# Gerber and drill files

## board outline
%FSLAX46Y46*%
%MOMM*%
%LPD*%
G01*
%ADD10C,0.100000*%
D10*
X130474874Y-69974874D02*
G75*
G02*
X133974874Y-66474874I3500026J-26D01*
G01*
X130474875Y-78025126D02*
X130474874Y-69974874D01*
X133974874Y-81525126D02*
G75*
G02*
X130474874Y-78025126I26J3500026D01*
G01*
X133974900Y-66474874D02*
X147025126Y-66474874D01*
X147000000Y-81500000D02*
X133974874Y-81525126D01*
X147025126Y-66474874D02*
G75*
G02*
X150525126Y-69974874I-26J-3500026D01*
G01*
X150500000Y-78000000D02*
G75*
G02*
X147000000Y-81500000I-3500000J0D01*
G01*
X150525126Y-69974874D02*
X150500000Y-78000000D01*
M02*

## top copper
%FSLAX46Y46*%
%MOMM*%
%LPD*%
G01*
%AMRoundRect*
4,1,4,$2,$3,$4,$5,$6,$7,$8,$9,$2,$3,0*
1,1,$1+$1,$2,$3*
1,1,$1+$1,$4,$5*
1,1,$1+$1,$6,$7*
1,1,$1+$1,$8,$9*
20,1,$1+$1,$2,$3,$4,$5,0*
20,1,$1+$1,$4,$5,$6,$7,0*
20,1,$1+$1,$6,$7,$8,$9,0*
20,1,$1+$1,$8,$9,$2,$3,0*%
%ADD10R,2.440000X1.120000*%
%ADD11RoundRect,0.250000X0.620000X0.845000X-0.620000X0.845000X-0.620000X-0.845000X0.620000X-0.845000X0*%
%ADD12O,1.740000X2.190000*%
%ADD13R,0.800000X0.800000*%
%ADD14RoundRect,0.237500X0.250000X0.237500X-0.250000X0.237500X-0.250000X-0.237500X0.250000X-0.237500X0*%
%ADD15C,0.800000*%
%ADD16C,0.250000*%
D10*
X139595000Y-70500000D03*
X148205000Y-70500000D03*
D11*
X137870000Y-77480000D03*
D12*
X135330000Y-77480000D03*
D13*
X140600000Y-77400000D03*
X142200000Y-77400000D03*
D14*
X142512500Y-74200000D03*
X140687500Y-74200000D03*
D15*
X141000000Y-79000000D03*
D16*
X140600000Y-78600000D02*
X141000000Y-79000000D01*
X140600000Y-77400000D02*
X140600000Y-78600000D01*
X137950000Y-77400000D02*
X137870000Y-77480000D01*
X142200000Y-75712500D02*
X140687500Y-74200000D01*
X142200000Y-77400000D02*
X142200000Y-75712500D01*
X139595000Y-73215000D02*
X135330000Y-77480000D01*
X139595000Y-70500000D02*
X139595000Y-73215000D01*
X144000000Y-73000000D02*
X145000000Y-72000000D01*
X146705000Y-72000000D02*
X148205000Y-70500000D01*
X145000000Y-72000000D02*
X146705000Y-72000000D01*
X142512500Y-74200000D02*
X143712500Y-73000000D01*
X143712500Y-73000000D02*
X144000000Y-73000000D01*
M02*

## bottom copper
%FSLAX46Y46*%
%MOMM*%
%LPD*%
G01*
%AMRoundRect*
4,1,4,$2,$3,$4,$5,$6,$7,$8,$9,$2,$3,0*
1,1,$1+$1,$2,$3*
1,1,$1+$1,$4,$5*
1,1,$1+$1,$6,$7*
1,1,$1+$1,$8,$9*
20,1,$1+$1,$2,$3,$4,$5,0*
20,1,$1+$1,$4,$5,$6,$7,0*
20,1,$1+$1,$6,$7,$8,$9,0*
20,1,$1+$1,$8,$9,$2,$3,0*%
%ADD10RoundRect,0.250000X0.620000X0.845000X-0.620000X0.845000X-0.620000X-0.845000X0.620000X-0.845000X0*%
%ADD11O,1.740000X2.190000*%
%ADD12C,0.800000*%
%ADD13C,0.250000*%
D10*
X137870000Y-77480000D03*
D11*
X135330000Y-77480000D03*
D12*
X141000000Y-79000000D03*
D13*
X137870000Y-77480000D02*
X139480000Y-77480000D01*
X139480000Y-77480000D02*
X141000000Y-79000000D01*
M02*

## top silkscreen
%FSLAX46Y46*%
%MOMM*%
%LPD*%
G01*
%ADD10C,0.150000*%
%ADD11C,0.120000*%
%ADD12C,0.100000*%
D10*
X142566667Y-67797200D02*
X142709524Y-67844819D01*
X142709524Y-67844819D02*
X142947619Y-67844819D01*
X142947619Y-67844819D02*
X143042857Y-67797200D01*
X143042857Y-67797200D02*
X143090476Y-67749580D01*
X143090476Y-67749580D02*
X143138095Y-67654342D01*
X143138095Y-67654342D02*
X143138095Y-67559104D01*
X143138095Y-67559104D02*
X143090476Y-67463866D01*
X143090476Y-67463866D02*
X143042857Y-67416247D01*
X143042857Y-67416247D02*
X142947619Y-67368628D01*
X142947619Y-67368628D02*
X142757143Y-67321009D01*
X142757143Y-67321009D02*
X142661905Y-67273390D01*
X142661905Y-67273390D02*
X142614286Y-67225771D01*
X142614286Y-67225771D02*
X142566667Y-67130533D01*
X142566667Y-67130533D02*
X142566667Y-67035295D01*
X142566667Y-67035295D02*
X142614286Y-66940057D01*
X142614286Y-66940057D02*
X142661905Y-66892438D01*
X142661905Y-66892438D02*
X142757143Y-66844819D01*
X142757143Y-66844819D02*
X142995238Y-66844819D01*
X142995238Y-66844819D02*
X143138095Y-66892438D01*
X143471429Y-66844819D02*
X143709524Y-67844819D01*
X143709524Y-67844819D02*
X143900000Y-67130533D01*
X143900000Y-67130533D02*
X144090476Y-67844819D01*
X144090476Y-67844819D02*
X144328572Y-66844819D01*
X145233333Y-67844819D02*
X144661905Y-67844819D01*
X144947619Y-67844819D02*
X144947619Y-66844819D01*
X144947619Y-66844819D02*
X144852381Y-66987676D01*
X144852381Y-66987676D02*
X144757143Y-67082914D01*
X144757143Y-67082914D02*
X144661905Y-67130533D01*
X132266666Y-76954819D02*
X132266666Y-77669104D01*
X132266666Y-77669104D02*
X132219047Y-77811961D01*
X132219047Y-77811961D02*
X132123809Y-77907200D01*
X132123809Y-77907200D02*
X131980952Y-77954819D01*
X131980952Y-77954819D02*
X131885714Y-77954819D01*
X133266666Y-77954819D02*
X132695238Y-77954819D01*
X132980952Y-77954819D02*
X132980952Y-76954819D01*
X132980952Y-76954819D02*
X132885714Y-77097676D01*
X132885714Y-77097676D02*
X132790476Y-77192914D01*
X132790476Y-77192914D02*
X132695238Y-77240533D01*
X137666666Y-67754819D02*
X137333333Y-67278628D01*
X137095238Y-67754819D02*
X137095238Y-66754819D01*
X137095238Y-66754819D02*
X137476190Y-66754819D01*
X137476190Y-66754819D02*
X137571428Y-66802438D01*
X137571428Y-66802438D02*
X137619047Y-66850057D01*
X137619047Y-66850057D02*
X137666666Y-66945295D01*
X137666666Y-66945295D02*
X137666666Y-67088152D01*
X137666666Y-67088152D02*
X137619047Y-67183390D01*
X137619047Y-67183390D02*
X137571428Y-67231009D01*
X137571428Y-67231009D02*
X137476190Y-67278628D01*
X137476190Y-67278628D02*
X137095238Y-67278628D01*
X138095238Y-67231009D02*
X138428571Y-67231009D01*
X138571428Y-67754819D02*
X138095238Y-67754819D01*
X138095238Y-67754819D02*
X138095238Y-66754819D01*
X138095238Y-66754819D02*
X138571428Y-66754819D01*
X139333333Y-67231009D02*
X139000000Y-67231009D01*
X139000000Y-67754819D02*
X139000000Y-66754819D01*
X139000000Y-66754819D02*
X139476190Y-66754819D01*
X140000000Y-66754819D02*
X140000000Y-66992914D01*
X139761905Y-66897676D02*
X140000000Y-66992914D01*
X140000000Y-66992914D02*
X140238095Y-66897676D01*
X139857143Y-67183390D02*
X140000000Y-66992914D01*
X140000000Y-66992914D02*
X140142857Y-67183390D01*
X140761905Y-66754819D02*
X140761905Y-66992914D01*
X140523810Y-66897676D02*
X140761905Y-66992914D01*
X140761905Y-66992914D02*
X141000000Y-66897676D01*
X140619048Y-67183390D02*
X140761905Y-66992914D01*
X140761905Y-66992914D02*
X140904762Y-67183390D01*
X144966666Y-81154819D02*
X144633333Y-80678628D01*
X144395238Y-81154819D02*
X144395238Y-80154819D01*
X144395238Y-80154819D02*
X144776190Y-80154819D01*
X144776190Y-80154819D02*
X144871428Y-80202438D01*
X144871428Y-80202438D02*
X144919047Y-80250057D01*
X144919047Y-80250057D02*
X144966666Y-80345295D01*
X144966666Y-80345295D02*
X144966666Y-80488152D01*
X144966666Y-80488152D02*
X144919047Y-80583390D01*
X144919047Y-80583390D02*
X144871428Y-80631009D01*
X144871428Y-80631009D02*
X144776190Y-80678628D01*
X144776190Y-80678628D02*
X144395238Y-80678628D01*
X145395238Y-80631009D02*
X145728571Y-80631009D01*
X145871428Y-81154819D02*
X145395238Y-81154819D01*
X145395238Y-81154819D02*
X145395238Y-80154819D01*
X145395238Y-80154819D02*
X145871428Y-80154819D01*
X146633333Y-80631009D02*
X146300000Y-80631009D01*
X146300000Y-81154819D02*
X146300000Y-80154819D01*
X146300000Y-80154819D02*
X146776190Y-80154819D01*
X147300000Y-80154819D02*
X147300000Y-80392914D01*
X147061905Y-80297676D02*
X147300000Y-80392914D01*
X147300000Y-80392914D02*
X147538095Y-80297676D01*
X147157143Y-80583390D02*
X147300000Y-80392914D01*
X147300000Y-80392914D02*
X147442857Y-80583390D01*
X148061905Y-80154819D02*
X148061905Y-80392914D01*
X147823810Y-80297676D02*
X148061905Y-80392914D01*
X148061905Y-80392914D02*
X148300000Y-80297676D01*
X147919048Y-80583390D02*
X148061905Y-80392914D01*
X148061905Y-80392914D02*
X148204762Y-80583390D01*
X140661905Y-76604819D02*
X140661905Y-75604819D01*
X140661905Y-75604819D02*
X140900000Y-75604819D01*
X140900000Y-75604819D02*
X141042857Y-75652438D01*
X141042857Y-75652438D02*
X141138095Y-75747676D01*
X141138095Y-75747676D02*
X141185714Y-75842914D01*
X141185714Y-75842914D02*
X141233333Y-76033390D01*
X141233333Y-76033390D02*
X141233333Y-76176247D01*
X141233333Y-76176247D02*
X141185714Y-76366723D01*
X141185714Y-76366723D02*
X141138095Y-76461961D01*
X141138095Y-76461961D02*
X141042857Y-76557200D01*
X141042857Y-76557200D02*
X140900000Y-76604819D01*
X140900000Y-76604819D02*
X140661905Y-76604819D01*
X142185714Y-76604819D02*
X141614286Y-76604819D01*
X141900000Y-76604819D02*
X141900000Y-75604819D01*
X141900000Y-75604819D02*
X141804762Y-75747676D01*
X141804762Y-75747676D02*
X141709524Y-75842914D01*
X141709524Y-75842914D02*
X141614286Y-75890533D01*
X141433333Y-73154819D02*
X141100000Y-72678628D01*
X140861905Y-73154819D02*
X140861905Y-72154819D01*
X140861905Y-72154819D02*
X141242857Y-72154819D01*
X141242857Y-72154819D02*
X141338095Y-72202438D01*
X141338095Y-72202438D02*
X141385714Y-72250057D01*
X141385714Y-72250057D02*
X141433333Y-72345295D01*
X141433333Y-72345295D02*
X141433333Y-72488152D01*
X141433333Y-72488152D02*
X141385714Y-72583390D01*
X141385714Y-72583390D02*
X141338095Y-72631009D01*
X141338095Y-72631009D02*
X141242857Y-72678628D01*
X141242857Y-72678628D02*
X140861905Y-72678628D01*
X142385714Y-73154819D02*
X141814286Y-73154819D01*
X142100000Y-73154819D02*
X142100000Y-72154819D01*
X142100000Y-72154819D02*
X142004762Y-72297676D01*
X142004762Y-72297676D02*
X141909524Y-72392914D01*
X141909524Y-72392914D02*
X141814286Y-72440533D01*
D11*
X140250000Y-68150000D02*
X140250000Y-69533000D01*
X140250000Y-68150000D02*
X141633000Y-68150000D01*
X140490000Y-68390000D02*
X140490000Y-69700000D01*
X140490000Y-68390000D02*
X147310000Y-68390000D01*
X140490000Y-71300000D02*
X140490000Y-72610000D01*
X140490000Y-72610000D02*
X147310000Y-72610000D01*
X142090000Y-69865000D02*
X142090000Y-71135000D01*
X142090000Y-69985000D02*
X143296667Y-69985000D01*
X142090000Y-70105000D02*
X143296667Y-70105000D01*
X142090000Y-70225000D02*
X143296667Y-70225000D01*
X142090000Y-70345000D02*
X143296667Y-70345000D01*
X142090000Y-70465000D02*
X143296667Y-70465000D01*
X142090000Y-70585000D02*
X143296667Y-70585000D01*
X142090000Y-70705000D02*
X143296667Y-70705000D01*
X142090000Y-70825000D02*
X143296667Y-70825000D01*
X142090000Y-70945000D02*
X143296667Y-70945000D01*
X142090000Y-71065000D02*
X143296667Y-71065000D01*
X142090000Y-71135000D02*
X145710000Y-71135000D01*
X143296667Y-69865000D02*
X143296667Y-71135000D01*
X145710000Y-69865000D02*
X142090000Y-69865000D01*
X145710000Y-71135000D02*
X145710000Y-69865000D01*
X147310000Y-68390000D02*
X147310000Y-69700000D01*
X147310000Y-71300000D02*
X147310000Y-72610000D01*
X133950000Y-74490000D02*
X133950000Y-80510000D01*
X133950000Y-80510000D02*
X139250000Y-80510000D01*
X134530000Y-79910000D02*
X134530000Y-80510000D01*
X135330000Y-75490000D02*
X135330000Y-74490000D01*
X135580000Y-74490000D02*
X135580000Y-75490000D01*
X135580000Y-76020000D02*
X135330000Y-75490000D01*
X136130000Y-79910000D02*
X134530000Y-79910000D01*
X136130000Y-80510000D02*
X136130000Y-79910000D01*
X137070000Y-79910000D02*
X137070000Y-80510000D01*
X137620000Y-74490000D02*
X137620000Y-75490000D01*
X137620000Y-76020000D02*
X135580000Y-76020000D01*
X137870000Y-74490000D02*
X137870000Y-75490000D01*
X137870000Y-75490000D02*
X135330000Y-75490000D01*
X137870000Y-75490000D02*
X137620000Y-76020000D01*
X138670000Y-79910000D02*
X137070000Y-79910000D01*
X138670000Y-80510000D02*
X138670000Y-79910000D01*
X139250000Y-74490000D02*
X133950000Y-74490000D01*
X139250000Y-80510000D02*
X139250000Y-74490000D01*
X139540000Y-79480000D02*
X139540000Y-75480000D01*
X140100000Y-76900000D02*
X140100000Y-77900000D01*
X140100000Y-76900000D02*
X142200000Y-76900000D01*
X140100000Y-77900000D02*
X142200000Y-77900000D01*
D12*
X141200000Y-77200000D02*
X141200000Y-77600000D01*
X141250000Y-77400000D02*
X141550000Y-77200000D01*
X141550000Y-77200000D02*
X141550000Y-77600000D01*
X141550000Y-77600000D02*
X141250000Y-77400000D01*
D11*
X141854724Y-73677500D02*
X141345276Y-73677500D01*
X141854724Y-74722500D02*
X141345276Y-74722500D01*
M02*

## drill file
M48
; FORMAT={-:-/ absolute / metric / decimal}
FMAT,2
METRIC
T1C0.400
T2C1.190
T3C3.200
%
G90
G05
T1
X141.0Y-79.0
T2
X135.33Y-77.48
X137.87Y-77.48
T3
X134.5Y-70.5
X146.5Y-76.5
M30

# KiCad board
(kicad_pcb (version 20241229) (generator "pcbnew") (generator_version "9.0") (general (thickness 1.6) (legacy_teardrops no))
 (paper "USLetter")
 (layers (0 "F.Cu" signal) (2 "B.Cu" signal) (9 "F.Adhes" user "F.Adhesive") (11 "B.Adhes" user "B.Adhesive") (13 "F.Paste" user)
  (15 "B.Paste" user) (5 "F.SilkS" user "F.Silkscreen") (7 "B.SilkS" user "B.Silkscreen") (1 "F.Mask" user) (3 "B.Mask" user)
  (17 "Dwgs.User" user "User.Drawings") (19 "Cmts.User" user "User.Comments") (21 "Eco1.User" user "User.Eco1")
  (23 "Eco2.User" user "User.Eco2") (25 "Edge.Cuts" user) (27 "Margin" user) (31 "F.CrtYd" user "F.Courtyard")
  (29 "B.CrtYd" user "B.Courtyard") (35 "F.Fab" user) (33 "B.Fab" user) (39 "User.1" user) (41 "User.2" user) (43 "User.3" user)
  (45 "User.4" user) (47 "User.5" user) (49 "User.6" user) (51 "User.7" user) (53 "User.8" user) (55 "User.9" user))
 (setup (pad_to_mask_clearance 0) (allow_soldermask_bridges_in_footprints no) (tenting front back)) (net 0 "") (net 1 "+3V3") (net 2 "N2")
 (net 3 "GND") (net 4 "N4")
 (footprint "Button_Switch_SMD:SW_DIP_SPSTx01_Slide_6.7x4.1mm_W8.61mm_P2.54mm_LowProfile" (layer "F.Cu") (at 143.9 70.5)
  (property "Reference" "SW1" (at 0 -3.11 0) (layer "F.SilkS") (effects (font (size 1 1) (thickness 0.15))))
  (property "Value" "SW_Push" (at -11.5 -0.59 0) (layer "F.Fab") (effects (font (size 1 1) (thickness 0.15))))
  (fp_line (start -3.65 -2.35) (end -3.65 -0.967) (stroke (width 0.12) (type solid)) (layer "F.SilkS"))
  (fp_line (start -3.65 -2.35) (end -2.267 -2.35) (stroke (width 0.12) (type solid)) (layer "F.SilkS"))
  (fp_line (start -3.41 -2.11) (end -3.41 -0.8) (stroke (width 0.12) (type solid)) (layer "F.SilkS"))
  (fp_line (start -3.41 -2.11) (end 3.41 -2.11) (stroke (width 0.12) (type solid)) (layer "F.SilkS"))
  (fp_line (start -3.41 0.8) (end -3.41 2.11) (stroke (width 0.12) (type solid)) (layer "F.SilkS"))
  (fp_line (start -3.41 2.11) (end 3.41 2.11) (stroke (width 0.12) (type solid)) (layer "F.SilkS"))
  (fp_line (start -1.81 -0.635) (end -1.81 0.635) (stroke (width 0.12) (type solid)) (layer "F.SilkS"))
  (fp_line (start -1.81 -0.515) (end -0.603333 -0.515) (stroke (width 0.12) (type solid)) (layer "F.SilkS"))
  (fp_line (start -1.81 -0.395) (end -0.603333 -0.395) (stroke (width 0.12) (type solid)) (layer "F.SilkS"))
  (fp_line (start -1.81 -0.275) (end -0.603333 -0.275) (stroke (width 0.12) (type solid)) (layer "F.SilkS"))
  (fp_line (start -1.81 -0.155) (end -0.603333 -0.155) (stroke (width 0.12) (type solid)) (layer "F.SilkS"))
  (fp_line (start -1.81 -0.035) (end -0.603333 -0.035) (stroke (width 0.12) (type solid)) (layer "F.SilkS"))
  (fp_line (start -1.81 0.085) (end -0.603333 0.085) (stroke (width 0.12) (type solid)) (layer "F.SilkS"))
  (fp_line (start -1.81 0.205) (end -0.603333 0.205) (stroke (width 0.12) (type solid)) (layer "F.SilkS"))
  (fp_line (start -1.81 0.325) (end -0.603333 0.325) (stroke (width 0.12) (type solid)) (layer "F.SilkS"))
  (fp_line (start -1.81 0.445) (end -0.603333 0.445) (stroke (width 0.12) (type solid)) (layer "F.SilkS"))
  (fp_line (start -1.81 0.565) (end -0.603333 0.565) (stroke (width 0.12) (type solid)) (layer "F.SilkS"))
  (fp_line (start -1.81 0.635) (end 1.81 0.635) (stroke (width 0.12) (type solid)) (layer "F.SilkS"))
  (fp_line (start -0.603333 -0.635) (end -0.603333 0.635) (stroke (width 0.12) (type solid)) (layer "F.SilkS"))
  (fp_line (start 1.81 -0.635) (end -1.81 -0.635) (stroke (width 0.12) (type solid)) (layer "F.SilkS"))
  (fp_line (start 1.81 0.635) (end 1.81 -0.635) (stroke (width 0.12) (type solid)) (layer "F.SilkS"))
  (fp_line (start 3.41 -2.11) (end 3.41 -0.8) (stroke (width 0.12) (type solid)) (layer "F.SilkS"))
  (fp_line (start 3.41 0.8) (end 3.41 2.11) (stroke (width 0.12) (type solid)) (layer "F.SilkS"))
  (pad "1" smd rect (at -4.305 0) (size 2.44 1.12) (layers "F.Cu" "F.Mask" "F.Paste") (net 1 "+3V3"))
  (pad "2" smd rect (at 4.305 0) (size 2.44 1.12) (layers "F.Cu" "F.Mask" "F.Paste") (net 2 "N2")))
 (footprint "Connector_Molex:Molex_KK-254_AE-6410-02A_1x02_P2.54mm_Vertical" (layer "F.Cu") (at 137.87 77.48 180)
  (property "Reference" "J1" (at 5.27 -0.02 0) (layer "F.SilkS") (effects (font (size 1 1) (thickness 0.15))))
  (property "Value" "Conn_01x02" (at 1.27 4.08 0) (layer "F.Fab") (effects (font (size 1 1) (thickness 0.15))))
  (fp_line (start 3.92 2.99) (end 3.92 -3.03) (stroke (width 0.12) (type solid)) (layer "F.SilkS"))
  (fp_line (start 3.92 -3.03) (end -1.38 -3.03) (stroke (width 0.12) (type solid)) (layer "F.SilkS"))
  (fp_line (start 3.34 -2.43) (end 3.34 -3.03) (stroke (width 0.12) (type solid)) (layer "F.SilkS"))
  (fp_line (start 2.54 1.99) (end 2.54 2.99) (stroke (width 0.12) (type solid)) (layer "F.SilkS"))
  (fp_line (start 2.29 2.99) (end 2.29 1.99) (stroke (width 0.12) (type solid)) (layer "F.SilkS"))
  (fp_line (start 2.29 1.46) (end 2.54 1.99) (stroke (width 0.12) (type solid)) (layer "F.SilkS"))
  (fp_line (start 1.74 -2.43) (end 3.34 -2.43) (stroke (width 0.12) (type solid)) (layer "F.SilkS"))
  (fp_line (start 1.74 -3.03) (end 1.74 -2.43) (stroke (width 0.12) (type solid)) (layer "F.SilkS"))
  (fp_line (start 0.8 -2.43) (end 0.8 -3.03) (stroke (width 0.12) (type solid)) (layer "F.SilkS"))
  (fp_line (start 0.25 2.99) (end 0.25 1.99) (stroke (width 0.12) (type solid)) (layer "F.SilkS"))
  (fp_line (start 0.25 1.46) (end 2.29 1.46) (stroke (width 0.12) (type solid)) (layer "F.SilkS"))
  (fp_line (start 0 2.99) (end 0 1.99) (stroke (width 0.12) (type solid)) (layer "F.SilkS"))
  (fp_line (start 0 1.99) (end 2.54 1.99) (stroke (width 0.12) (type solid)) (layer "F.SilkS"))
  (fp_line (start 0 1.99) (end 0.25 1.46) (stroke (width 0.12) (type solid)) (layer "F.SilkS"))
  (fp_line (start -0.8 -2.43) (end 0.8 -2.43) (stroke (width 0.12) (type solid)) (layer "F.SilkS"))
  (fp_line (start -0.8 -3.03) (end -0.8 -2.43) (stroke (width 0.12) (type solid)) (layer "F.SilkS"))
  (fp_line (start -1.38 2.99) (end 3.92 2.99) (stroke (width 0.12) (type solid)) (layer "F.SilkS"))
  (fp_line (start -1.38 -3.03) (end -1.38 2.99) (stroke (width 0.12) (type solid)) (layer "F.SilkS"))
  (fp_line (start -1.67 -2) (end -1.67 2) (stroke (width 0.12) (type solid)) (layer "F.SilkS"))
  (pad "1" thru_hole roundrect (at 0 0 180) (size 1.74 2.19) (drill 1.19) (layers "*.Cu" "*.Mask") (remove_unused_layers no)
   (roundrect_rratio 0.143678) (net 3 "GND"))
  (pad "2" thru_hole oval (at 2.54 0 180) (size 1.74 2.19) (drill 1.19) (layers "*.Cu" "*.Mask") (remove_unused_layers no) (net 1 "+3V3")))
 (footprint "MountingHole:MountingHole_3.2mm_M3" (layer "F.Cu") (at 134.5 70.5)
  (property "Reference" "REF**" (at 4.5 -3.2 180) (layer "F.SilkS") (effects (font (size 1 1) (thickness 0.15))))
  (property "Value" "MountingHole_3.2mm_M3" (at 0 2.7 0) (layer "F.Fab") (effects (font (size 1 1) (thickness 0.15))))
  (pad "" np_thru_hole circle (at 0 0) (size 3.2 3.2) (drill 3.2) (layers "*.Cu" "*.Mask")))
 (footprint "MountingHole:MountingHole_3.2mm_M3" (layer "F.Cu") (at 146.5 76.5)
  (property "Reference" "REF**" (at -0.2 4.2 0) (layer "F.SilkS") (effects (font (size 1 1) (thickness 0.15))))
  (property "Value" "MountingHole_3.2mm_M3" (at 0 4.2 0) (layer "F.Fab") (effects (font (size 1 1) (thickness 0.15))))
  (pad "" np_thru_hole circle (at 0 0) (size 3.2 3.2) (drill 3.2) (layers "*.Cu" "*.Mask")))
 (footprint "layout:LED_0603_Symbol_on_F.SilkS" (layer "F.Cu") (at 141.4 77.4)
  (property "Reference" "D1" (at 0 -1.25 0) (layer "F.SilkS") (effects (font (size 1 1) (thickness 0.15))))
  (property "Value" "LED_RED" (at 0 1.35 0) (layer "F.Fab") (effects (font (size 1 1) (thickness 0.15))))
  (fp_line (start -1.3 -0.5) (end -1.3 0.5) (stroke (width 0.12) (type solid)) (layer "F.SilkS"))
  (fp_line (start -1.3 -0.5) (end 0.8 -0.5) (stroke (width 0.12) (type solid)) (layer "F.SilkS"))
  (fp_line (start -1.3 0.5) (end 0.8 0.5) (stroke (width 0.12) (type solid)) (layer "F.SilkS"))
  (fp_line (start -0.2 -0.2) (end -0.2 0.2) (stroke (width 0.1) (type solid)) (layer "F.SilkS"))
  (fp_line (start -0.15 0) (end 0.15 -0.2) (stroke (width 0.1) (type solid)) (layer "F.SilkS"))
  (fp_line (start 0.15 -0.2) (end 0.15 0.2) (stroke (width 0.1) (type solid)) (layer "F.SilkS"))
  (fp_line (start 0.15 0.2) (end -0.15 0) (stroke (width 0.1) (type solid)) (layer "F.SilkS"))
  (pad "1" smd rect (at -0.8 0 180) (size 0.8 0.8) (layers "F.Cu" "F.Mask" "F.Paste") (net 3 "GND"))
  (pad "2" smd rect (at 0.8 0 180) (size 0.8 0.8) (layers "F.Cu" "F.Mask" "F.Paste") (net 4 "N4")))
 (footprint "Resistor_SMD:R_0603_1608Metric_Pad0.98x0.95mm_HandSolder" (layer "F.Cu") (at 141.6 74.2 180)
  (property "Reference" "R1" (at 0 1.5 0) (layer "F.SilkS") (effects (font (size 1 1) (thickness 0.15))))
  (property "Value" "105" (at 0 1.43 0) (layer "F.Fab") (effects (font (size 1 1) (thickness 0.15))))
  (fp_line (start -0.254724 0.5225) (end 0.254724 0.5225) (stroke (width 0.12) (type solid)) (layer "F.SilkS"))
  (fp_line (start -0.254724 -0.5225) (end 0.254724 -0.5225) (stroke (width 0.12) (type solid)) (layer "F.SilkS"))
  (pad "1" smd roundrect (at -0.9125 0 180) (size 0.975 0.95) (layers "F.Cu" "F.Mask" "F.Paste") (roundrect_rratio 0.25) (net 2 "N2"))
  (pad "2" smd roundrect (at 0.9125 0 180) (size 0.975 0.95) (layers "F.Cu" "F.Mask" "F.Paste") (roundrect_rratio 0.25) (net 4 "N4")))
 (gr_arc (start 130.474874 69.974874) (mid 131.5 67.5) (end 133.974874 66.474874) (stroke (width 0.1) (type default)) (layer "Edge.Cuts"))
 (gr_line (start 130.474875 78.025126) (end 130.474874 69.974874) (stroke (width 0.1) (type default)) (layer "Edge.Cuts"))
 (gr_arc (start 133.974874 81.525126) (mid 131.5 80.5) (end 130.474874 78.025126) (stroke (width 0.1) (type default)) (layer "Edge.Cuts"))
 (gr_line (start 133.9749 66.474874) (end 147.025126 66.474874) (stroke (width 0.1) (type default)) (layer "Edge.Cuts"))
 (gr_line (start 147 81.5) (end 133.974874 81.525126) (stroke (width 0.1) (type default)) (layer "Edge.Cuts"))
 (gr_arc (start 147.025126 66.474874) (mid 149.5 67.5) (end 150.525126 69.974874) (stroke (width 0.1) (type default)) (layer "Edge.Cuts"))
 (gr_arc (start 150.5 78) (mid 149.474874 80.474874) (end 147 81.5) (stroke (width 0.1) (type default)) (layer "Edge.Cuts"))
 (gr_line (start 150.525126 69.974874) (end 150.5 78) (stroke (width 0.1) (type default)) (layer "Edge.Cuts"))
 (segment (start 140.6 78.6) (end 141 79) (width 0.25) (layer "F.Cu") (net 3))
 (segment (start 140.6 77.4) (end 140.6 78.6) (width 0.25) (layer "F.Cu") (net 3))
 (segment (start 137.95 77.4) (end 137.87 77.48) (width 0.25) (layer "F.Cu") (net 3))
 (via (at 141 79) (size 0.8) (drill 0.4) (layers "F.Cu" "B.Cu") (free yes) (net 3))
 (segment (start 137.87 77.48) (end 139.48 77.48) (width 0.25) (layer "B.Cu") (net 3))
 (segment (start 139.48 77.48) (end 141 79) (width 0.25) (layer "B.Cu") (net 3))
 (segment (start 142.2 75.7125) (end 140.6875 74.2) (width 0.25) (layer "F.Cu") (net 4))
 (segment (start 142.2 77.4) (end 142.2 75.7125) (width 0.25) (layer "F.Cu") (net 4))
 (segment (start 139.595 73.215) (end 135.33 77.48) (width 0.25) (layer "F.Cu") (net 1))
 (segment (start 139.595 70.5) (end 139.595 73.215) (width 0.25) (layer "F.Cu") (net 1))
 (segment (start 144 73) (end 145 72) (width 0.25) (layer "F.Cu") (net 2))
 (segment (start 146.705 72) (end 148.205 70.5) (width 0.25) (layer "F.Cu") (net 2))
 (segment (start 145 72) (end 146.705 72) (width 0.25) (layer "F.Cu") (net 2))
 (segment (start 142.5125 74.2) (end 143.7125 73) (width 0.25) (layer "F.Cu") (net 2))
 (segment (start 143.7125 73) (end 144 73) (width 0.25) (layer "F.Cu") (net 2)))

